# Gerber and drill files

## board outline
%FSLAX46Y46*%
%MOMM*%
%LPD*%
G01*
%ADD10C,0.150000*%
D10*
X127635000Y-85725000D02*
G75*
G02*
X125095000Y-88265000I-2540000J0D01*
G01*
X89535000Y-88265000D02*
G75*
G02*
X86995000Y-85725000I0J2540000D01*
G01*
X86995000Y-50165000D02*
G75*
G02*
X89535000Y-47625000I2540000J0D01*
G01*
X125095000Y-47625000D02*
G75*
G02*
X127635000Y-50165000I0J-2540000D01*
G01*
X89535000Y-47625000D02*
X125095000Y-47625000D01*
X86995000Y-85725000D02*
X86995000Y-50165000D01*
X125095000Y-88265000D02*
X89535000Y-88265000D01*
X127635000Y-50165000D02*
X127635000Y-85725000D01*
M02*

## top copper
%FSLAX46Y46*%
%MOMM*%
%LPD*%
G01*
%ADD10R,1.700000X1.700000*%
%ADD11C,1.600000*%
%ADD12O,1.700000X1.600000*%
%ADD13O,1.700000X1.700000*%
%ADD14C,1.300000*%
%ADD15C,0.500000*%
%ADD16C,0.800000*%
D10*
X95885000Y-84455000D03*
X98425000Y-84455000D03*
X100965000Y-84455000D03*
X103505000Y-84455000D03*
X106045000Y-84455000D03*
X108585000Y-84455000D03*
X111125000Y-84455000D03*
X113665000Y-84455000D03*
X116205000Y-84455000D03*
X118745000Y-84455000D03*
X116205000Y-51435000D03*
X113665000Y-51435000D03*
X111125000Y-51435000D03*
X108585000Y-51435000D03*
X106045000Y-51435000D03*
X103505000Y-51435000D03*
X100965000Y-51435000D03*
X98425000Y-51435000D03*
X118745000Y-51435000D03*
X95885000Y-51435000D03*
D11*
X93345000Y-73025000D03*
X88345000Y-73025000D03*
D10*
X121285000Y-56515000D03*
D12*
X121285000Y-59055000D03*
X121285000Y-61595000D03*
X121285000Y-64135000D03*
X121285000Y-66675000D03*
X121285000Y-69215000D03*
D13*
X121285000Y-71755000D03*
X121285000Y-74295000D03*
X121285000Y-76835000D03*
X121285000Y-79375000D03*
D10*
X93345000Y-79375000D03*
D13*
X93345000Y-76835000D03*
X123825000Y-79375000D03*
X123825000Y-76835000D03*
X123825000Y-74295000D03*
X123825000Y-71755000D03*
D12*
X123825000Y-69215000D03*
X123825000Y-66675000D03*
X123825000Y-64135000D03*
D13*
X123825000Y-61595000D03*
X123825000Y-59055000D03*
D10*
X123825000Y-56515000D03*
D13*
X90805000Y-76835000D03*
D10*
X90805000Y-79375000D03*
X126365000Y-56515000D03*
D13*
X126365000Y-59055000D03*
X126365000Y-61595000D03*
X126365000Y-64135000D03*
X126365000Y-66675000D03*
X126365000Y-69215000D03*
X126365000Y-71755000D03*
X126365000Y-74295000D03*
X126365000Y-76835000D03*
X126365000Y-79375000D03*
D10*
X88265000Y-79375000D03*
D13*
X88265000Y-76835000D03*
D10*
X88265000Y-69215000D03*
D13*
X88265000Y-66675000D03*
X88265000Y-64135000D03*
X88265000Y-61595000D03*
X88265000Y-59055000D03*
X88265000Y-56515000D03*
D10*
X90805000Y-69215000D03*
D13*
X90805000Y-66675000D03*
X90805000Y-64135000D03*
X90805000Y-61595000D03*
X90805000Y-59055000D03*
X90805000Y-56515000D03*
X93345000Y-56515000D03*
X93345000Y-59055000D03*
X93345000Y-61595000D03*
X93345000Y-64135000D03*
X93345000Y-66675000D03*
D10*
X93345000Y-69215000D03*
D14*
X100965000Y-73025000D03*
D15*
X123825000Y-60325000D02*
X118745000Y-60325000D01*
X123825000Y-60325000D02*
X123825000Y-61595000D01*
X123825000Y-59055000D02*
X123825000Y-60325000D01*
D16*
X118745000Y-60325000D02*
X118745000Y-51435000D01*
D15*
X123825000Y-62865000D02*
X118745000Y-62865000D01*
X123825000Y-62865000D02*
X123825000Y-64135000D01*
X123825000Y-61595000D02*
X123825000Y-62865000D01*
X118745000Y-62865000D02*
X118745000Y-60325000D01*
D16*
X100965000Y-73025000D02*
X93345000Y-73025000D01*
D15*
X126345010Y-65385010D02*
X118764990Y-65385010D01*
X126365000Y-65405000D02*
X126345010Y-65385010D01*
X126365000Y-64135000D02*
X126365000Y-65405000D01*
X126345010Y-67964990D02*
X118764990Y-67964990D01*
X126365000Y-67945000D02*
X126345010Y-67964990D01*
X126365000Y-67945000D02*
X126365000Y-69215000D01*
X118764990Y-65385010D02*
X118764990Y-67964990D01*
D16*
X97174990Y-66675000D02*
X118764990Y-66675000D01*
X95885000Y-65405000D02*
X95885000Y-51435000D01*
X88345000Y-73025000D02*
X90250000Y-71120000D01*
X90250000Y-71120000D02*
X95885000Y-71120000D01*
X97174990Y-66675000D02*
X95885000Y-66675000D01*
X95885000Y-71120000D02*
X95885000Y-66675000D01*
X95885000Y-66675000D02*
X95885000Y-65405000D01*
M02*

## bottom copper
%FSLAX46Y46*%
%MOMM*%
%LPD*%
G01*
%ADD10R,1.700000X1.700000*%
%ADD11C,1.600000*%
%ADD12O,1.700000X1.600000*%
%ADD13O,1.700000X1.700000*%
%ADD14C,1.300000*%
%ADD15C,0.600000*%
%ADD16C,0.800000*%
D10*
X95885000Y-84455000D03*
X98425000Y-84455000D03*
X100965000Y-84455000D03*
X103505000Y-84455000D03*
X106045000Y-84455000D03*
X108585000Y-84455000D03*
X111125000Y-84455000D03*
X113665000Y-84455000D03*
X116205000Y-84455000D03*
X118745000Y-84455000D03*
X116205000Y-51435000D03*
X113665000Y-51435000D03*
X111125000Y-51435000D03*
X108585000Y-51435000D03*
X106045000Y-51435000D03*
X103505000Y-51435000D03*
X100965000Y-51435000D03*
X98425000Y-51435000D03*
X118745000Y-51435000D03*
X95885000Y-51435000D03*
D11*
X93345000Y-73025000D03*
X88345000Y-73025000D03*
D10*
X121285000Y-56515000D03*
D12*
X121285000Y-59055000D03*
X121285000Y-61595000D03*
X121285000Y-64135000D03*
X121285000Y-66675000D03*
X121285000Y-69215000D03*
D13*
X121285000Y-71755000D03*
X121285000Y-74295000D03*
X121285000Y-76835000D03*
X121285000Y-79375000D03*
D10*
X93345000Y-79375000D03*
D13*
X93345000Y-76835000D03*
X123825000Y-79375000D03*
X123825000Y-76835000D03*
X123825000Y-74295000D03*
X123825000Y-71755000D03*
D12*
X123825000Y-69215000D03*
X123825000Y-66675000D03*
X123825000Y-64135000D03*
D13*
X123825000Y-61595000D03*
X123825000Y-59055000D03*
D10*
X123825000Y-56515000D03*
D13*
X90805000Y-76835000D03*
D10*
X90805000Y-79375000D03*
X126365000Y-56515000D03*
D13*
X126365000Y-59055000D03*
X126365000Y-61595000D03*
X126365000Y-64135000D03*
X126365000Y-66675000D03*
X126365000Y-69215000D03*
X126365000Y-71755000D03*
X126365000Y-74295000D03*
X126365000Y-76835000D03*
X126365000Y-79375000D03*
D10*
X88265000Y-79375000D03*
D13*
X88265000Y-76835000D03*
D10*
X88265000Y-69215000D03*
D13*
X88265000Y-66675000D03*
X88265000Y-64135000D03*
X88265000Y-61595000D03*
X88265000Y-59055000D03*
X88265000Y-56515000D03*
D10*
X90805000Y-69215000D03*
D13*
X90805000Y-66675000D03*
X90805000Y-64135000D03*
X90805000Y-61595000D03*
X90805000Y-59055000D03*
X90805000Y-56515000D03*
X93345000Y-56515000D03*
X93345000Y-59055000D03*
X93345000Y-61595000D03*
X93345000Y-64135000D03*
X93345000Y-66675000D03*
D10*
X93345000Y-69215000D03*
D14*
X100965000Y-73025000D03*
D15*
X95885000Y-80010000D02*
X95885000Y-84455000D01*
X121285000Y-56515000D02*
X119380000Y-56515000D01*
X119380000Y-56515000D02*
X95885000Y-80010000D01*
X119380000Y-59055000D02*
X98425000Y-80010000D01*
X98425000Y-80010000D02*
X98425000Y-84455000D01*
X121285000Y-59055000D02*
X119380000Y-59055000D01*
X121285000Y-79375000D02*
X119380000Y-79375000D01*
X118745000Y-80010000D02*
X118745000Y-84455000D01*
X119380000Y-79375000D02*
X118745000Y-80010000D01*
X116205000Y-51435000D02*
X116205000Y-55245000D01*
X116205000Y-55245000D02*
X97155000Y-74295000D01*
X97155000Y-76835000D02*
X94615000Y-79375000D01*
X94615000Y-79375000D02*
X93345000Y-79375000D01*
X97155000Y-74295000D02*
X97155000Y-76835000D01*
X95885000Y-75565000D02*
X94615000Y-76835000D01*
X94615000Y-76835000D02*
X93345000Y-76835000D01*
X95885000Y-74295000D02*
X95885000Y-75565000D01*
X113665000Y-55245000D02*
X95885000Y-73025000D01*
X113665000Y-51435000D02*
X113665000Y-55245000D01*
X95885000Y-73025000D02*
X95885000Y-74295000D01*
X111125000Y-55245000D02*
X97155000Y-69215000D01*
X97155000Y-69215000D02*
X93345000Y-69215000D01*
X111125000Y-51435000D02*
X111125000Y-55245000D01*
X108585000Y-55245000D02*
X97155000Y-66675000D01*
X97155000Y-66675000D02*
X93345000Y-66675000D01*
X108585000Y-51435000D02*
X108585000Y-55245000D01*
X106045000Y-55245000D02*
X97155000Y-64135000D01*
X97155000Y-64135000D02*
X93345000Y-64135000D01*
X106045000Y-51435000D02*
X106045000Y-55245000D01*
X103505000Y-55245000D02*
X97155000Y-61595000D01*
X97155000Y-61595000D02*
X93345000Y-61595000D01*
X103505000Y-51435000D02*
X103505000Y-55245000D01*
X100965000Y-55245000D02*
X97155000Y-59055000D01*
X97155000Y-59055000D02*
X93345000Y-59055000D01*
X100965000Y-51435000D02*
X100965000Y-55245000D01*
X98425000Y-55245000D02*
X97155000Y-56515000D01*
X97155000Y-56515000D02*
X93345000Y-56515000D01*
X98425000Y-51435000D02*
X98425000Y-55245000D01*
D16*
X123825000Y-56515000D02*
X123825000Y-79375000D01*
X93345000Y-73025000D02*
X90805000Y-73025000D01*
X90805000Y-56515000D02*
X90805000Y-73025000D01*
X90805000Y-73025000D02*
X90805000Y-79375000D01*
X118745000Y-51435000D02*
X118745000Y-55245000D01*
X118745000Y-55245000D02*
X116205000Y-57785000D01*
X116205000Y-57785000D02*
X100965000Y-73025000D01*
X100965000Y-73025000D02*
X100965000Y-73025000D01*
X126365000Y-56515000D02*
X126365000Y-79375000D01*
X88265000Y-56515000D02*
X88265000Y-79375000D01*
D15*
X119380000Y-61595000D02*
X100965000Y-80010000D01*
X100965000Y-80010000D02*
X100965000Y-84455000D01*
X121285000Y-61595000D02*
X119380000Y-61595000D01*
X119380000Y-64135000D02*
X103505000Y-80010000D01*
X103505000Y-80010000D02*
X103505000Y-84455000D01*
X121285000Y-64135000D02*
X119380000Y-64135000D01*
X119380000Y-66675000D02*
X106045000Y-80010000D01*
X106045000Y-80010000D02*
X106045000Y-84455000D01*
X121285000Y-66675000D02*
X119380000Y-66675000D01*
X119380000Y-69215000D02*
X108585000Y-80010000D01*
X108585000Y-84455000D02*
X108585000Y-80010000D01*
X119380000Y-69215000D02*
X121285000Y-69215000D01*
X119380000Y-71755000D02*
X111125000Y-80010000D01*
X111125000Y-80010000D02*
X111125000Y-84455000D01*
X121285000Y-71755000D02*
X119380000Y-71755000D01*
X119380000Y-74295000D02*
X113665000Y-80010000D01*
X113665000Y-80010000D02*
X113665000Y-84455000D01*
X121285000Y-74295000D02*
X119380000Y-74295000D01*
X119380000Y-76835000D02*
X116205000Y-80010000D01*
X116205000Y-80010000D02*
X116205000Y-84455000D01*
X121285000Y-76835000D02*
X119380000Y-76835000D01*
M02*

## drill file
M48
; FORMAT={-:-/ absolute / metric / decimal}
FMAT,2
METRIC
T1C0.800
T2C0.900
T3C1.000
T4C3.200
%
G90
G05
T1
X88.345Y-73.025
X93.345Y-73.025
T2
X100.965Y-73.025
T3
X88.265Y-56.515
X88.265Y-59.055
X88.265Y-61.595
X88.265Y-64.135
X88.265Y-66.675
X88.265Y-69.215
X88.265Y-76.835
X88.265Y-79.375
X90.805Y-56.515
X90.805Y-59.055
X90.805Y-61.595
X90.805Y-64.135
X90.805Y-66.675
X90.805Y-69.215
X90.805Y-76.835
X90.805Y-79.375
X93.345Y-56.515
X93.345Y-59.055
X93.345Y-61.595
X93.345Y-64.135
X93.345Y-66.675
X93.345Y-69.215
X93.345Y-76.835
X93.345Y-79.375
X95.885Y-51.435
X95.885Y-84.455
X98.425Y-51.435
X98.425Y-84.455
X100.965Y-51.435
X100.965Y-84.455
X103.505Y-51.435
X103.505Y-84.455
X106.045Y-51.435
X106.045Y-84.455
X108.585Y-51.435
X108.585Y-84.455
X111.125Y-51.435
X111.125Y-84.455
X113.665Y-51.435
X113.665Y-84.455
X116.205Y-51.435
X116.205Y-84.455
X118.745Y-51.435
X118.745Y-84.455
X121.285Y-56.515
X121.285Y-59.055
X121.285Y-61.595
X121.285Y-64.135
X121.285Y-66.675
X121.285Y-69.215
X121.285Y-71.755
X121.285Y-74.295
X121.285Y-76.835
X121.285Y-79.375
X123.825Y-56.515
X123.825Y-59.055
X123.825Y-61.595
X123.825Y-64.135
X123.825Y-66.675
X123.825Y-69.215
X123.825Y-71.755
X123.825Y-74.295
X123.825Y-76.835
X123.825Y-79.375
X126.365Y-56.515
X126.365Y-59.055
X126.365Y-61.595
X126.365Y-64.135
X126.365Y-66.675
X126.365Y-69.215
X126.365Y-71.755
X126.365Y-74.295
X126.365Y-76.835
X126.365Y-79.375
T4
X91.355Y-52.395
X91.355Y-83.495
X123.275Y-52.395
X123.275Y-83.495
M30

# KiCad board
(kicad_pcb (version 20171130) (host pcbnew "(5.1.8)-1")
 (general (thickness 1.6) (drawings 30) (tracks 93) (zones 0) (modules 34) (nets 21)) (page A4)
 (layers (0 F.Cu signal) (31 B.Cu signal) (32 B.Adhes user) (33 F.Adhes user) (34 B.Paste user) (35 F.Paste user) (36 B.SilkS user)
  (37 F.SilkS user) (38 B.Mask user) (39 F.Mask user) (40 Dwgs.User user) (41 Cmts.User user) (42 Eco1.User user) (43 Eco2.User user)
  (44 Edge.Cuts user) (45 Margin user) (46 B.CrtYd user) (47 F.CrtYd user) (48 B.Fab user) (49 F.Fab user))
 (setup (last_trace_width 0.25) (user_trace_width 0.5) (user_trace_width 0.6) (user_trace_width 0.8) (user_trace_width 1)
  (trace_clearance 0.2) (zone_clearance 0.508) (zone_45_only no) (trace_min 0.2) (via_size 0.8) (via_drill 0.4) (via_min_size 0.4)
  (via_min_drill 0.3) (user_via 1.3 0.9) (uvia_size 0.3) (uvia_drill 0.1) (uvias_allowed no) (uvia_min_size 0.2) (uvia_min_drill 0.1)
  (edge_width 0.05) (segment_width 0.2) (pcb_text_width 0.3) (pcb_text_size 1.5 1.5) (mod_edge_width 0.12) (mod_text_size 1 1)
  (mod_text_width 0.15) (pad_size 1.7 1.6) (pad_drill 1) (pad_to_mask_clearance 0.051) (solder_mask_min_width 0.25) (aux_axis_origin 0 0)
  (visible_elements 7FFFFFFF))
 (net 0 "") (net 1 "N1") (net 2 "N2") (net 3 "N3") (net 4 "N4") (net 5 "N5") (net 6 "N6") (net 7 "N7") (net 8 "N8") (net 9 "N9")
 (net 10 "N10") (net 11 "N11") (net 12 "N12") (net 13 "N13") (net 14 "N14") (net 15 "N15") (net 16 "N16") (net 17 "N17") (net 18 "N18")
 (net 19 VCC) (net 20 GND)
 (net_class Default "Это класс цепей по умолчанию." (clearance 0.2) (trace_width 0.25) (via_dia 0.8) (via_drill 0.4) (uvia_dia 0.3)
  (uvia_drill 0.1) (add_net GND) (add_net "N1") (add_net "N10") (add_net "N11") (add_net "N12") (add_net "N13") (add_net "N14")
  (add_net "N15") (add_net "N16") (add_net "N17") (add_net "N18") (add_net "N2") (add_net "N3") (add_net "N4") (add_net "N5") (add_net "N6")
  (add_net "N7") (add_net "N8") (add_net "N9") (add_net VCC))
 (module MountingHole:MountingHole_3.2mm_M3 (layer F.Cu) (at 123.2750 52.3950)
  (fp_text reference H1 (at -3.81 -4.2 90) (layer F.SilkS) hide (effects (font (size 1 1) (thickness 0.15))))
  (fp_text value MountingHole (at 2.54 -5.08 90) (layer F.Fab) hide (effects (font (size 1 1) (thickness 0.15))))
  (pad 1 np_thru_hole circle (at 0 0 270) (size 3.2 3.2) (drill 3.2) (layers *.Cu *.Mask)))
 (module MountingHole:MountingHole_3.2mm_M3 (layer F.Cu) (at 91.3550 52.3950)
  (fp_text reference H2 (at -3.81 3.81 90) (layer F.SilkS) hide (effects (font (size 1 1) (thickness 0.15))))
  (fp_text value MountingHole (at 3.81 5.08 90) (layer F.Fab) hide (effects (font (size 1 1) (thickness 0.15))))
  (pad 1 np_thru_hole circle (at 0 0 270) (size 3.2 3.2) (drill 3.2) (layers *.Cu *.Mask)))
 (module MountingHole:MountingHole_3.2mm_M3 (layer F.Cu) (at 123.2750 83.4950)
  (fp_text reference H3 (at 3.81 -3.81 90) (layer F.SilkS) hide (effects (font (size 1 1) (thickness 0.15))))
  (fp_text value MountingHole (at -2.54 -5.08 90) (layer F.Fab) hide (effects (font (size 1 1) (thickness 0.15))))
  (pad 1 np_thru_hole circle (at 0 0 270) (size 3.2 3.2) (drill 3.2) (layers *.Cu *.Mask)))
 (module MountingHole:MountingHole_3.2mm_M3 (layer F.Cu) (at 91.3550 83.4950)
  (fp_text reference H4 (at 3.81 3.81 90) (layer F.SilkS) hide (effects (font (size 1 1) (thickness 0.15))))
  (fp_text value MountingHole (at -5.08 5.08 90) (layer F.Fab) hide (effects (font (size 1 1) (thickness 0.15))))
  (pad 1 np_thru_hole circle (at 0 0 270) (size 3.2 3.2) (drill 3.2) (layers *.Cu *.Mask)))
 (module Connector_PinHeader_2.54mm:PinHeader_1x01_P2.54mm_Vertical (layer F.Cu) (at 95.885 84.455 270)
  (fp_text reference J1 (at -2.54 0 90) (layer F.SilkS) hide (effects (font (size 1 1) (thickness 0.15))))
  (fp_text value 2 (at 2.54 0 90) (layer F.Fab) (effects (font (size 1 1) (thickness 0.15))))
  (pad 1 thru_hole rect (at 0 0 270) (size 1.7 1.7) (drill 1) (layers *.Cu *.Mask) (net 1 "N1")))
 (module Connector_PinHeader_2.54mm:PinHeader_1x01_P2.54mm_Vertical (layer F.Cu) (at 98.425 84.455 270)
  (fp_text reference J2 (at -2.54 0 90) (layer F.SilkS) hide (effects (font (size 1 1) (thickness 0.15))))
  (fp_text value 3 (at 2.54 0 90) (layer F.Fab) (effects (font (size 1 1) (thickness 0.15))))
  (pad 1 thru_hole rect (at 0 0 270) (size 1.7 1.7) (drill 1) (layers *.Cu *.Mask) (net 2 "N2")))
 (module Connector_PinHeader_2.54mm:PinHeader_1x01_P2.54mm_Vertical (layer F.Cu) (at 100.965 84.455 270)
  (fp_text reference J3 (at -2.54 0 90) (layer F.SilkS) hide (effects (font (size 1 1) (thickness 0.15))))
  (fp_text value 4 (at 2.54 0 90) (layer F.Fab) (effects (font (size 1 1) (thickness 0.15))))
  (pad 1 thru_hole rect (at 0 0 270) (size 1.7 1.7) (drill 1) (layers *.Cu *.Mask) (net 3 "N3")))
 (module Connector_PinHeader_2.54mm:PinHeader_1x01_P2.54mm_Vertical (layer F.Cu) (at 103.505 84.455 270)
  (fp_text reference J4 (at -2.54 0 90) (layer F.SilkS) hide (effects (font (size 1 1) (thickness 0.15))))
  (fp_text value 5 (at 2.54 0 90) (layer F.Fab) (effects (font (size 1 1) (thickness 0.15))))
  (pad 1 thru_hole rect (at 0 0 270) (size 1.7 1.7) (drill 1) (layers *.Cu *.Mask) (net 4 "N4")))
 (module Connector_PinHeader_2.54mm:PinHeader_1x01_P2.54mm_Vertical (layer F.Cu) (at 106.045 84.455 270)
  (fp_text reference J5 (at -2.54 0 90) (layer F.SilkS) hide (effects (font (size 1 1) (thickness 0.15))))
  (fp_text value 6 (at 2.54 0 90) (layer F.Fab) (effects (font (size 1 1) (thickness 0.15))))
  (pad 1 thru_hole rect (at 0 0 270) (size 1.7 1.7) (drill 1) (layers *.Cu *.Mask) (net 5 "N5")))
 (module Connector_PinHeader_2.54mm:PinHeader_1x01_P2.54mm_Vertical (layer F.Cu) (at 108.585 84.455 270)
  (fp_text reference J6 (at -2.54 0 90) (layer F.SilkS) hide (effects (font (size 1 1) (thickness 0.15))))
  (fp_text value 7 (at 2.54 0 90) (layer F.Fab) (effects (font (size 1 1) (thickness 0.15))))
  (pad 1 thru_hole rect (at 0 0 270) (size 1.7 1.7) (drill 1) (layers *.Cu *.Mask) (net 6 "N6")))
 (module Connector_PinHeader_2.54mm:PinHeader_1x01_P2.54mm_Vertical (layer F.Cu) (at 111.125 84.455 270)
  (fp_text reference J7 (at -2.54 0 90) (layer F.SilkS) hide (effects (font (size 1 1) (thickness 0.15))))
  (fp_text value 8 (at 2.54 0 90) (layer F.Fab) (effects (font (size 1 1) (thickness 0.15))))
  (pad 1 thru_hole rect (at 0 0 270) (size 1.7 1.7) (drill 1) (layers *.Cu *.Mask) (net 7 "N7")))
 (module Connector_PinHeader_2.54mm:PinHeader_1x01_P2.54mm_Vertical (layer F.Cu) (at 113.665 84.455 270)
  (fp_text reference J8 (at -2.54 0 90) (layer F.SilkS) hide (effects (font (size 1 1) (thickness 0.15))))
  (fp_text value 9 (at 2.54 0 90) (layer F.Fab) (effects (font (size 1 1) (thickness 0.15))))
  (pad 1 thru_hole rect (at 0 0 270) (size 1.7 1.7) (drill 1) (layers *.Cu *.Mask) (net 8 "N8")))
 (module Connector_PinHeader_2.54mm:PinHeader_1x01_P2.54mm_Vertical (layer F.Cu) (at 116.205 84.455 270)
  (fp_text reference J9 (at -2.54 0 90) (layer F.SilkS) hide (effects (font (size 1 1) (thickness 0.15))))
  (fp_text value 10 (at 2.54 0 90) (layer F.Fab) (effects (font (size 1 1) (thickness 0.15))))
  (pad 1 thru_hole rect (at 0 0 270) (size 1.7 1.7) (drill 1) (layers *.Cu *.Mask) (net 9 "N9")))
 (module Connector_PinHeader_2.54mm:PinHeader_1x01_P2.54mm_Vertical (layer F.Cu) (at 118.745 84.455 270)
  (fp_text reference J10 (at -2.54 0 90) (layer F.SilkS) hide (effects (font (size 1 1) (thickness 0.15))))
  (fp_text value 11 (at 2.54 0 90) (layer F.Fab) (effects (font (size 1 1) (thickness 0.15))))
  (pad 1 thru_hole rect (at 0 0 270) (size 1.7 1.7) (drill 1) (layers *.Cu *.Mask) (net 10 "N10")))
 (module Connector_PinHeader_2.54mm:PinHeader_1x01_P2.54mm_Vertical (layer F.Cu) (at 116.205 51.435 270)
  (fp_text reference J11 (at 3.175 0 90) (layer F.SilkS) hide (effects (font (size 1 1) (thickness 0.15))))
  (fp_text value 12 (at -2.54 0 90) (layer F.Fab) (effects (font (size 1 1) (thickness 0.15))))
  (pad 1 thru_hole rect (at 0 0 270) (size 1.7 1.7) (drill 1) (layers *.Cu *.Mask) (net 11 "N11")))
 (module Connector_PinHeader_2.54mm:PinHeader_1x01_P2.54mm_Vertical (layer F.Cu) (at 113.665 51.435 270)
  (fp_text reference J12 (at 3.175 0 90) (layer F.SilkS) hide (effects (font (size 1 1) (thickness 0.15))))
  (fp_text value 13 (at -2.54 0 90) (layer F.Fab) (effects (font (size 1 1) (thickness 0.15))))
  (pad 1 thru_hole rect (at 0 0 270) (size 1.7 1.7) (drill 1) (layers *.Cu *.Mask) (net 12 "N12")))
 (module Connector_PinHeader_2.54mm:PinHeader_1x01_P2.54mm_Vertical (layer F.Cu) (at 111.125 51.435 270)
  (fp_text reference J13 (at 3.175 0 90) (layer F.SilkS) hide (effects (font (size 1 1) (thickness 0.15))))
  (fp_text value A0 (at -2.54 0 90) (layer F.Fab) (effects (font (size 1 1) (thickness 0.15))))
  (pad 1 thru_hole rect (at 0 0 270) (size 1.7 1.7) (drill 1) (layers *.Cu *.Mask) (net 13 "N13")))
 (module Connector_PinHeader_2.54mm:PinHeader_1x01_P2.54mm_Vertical (layer F.Cu) (at 108.585 51.435 270)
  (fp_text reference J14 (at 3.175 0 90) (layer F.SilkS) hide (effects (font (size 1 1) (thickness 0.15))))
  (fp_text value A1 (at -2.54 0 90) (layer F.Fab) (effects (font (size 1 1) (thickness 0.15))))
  (pad 1 thru_hole rect (at 0 0 270) (size 1.7 1.7) (drill 1) (layers *.Cu *.Mask) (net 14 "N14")))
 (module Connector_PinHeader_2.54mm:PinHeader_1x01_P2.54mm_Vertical (layer F.Cu) (at 106.045 51.435 270)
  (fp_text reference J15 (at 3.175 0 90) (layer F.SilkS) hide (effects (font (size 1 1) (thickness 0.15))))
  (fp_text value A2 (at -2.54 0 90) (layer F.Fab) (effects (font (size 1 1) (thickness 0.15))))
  (pad 1 thru_hole rect (at 0 0 270) (size 1.7 1.7) (drill 1) (layers *.Cu *.Mask) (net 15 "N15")))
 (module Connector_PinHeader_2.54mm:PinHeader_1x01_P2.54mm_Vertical (layer F.Cu) (at 103.505 51.435 270)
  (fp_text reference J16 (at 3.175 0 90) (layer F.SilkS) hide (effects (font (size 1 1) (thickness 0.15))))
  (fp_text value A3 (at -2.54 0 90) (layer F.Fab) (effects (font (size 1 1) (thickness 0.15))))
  (pad 1 thru_hole rect (at 0 0 270) (size 1.7 1.7) (drill 1) (layers *.Cu *.Mask) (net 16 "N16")))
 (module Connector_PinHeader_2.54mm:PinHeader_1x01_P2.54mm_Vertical (layer F.Cu) (at 100.965 51.435 270)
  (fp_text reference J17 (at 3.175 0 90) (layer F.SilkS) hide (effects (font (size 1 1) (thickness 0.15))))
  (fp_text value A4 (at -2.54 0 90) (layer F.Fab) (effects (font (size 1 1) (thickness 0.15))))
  (pad 1 thru_hole rect (at 0 0 270) (size 1.7 1.7) (drill 1) (layers *.Cu *.Mask) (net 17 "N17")))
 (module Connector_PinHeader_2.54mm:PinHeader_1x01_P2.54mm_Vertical (layer F.Cu) (at 98.425 51.435 270)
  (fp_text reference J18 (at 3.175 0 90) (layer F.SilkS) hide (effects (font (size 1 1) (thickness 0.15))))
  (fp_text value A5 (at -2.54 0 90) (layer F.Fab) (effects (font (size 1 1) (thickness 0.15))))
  (pad 1 thru_hole rect (at 0 0 270) (size 1.7 1.7) (drill 1) (layers *.Cu *.Mask) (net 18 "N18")))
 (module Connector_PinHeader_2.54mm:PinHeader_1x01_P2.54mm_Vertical (layer F.Cu) (at 118.745 51.435 270)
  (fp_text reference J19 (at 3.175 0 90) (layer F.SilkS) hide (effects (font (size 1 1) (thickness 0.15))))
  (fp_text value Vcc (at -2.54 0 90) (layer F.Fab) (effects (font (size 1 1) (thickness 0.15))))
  (pad 1 thru_hole rect (at 0 0 270) (size 1.7 1.7) (drill 1) (layers *.Cu *.Mask) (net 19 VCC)))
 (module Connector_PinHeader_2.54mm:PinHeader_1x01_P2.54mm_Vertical (layer F.Cu) (at 95.885 51.435 270)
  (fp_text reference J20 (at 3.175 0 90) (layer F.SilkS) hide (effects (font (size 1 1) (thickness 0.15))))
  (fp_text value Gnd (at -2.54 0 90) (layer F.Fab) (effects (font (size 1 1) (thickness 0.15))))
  (pad 1 thru_hole rect (at 0 0 270) (size 1.7 1.7) (drill 1) (layers *.Cu *.Mask) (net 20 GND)))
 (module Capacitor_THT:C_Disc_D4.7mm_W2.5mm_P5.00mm (layer F.Cu) (at 93.345 73.025 180)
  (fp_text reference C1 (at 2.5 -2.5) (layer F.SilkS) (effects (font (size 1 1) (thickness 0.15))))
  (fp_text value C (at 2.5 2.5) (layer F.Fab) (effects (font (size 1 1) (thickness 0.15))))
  (pad 1 thru_hole circle (at 0 0 180) (size 1.6 1.6) (drill 0.8) (layers *.Cu *.Mask) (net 19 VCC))
  (pad 2 thru_hole circle (at 5 0 180) (size 1.6 1.6) (drill 0.8) (layers *.Cu *.Mask) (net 20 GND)))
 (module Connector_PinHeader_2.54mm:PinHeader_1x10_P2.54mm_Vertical (layer F.Cu) (at 121.285 56.515)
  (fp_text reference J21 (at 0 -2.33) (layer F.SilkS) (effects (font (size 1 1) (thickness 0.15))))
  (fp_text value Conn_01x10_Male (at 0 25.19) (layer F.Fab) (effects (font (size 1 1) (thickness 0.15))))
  (pad 1 thru_hole rect (at 0 0) (size 1.7 1.7) (drill 1) (layers *.Cu *.Mask) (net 1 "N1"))
  (pad 2 thru_hole oval (at 0 2.54) (size 1.7 1.6) (drill 1) (layers *.Cu *.Mask) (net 2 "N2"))
  (pad 3 thru_hole oval (at 0 5.08) (size 1.7 1.6) (drill 1) (layers *.Cu *.Mask) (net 3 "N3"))
  (pad 4 thru_hole oval (at 0 7.62) (size 1.7 1.6) (drill 1) (layers *.Cu *.Mask) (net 4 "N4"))
  (pad 5 thru_hole oval (at 0 10.16) (size 1.7 1.6) (drill 1) (layers *.Cu *.Mask) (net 5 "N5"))
  (pad 6 thru_hole oval (at 0 12.7) (size 1.7 1.6) (drill 1) (layers *.Cu *.Mask) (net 6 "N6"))
  (pad 7 thru_hole oval (at 0 15.24) (size 1.7 1.7) (drill 1) (layers *.Cu *.Mask) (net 7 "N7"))
  (pad 8 thru_hole oval (at 0 17.78) (size 1.7 1.7) (drill 1) (layers *.Cu *.Mask) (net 8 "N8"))
  (pad 9 thru_hole oval (at 0 20.32) (size 1.7 1.7) (drill 1) (layers *.Cu *.Mask) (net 9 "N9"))
  (pad 10 thru_hole oval (at 0 22.86) (size 1.7 1.7) (drill 1) (layers *.Cu *.Mask) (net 10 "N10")))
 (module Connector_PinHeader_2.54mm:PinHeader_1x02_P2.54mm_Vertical (layer F.Cu) (at 93.345 79.375 180)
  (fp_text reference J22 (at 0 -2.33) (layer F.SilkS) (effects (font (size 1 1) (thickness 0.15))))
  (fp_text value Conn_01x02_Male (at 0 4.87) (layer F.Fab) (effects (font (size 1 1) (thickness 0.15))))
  (pad 1 thru_hole rect (at 0 0 180) (size 1.7 1.7) (drill 1) (layers *.Cu *.Mask) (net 11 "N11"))
  (pad 2 thru_hole oval (at 0 2.54 180) (size 1.7 1.7) (drill 1) (layers *.Cu *.Mask) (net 12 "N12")))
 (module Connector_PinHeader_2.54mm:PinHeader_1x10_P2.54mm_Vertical (layer F.Cu) (at 123.825 56.515)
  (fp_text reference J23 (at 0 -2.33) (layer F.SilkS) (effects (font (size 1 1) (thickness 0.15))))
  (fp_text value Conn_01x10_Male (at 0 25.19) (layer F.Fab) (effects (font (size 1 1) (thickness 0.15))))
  (pad 10 thru_hole oval (at 0 22.86) (size 1.7 1.7) (drill 1) (layers *.Cu *.Mask) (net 19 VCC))
  (pad 9 thru_hole oval (at 0 20.32) (size 1.7 1.7) (drill 1) (layers *.Cu *.Mask) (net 19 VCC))
  (pad 8 thru_hole oval (at 0 17.78) (size 1.7 1.7) (drill 1) (layers *.Cu *.Mask) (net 19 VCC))
  (pad 7 thru_hole oval (at 0 15.24) (size 1.7 1.7) (drill 1) (layers *.Cu *.Mask) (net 19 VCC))
  (pad 6 thru_hole oval (at 0 12.7) (size 1.7 1.6) (drill 1) (layers *.Cu *.Mask) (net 19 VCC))
  (pad 5 thru_hole oval (at 0 10.16) (size 1.7 1.6) (drill 1) (layers *.Cu *.Mask) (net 19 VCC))
  (pad 4 thru_hole oval (at 0 7.62) (size 1.7 1.6) (drill 1) (layers *.Cu *.Mask) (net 19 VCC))
  (pad 3 thru_hole oval (at 0 5.08) (size 1.7 1.7) (drill 1) (layers *.Cu *.Mask) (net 19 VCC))
  (pad 2 thru_hole oval (at 0 2.54) (size 1.7 1.7) (drill 1) (layers *.Cu *.Mask) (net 19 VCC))
  (pad 1 thru_hole rect (at 0 0) (size 1.7 1.7) (drill 1) (layers *.Cu *.Mask) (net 19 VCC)))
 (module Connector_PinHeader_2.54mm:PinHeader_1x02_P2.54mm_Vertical (layer F.Cu) (at 90.805 79.375 180)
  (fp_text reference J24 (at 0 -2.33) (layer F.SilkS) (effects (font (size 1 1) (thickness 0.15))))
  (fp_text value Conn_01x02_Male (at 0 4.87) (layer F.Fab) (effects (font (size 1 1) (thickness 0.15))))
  (pad 2 thru_hole oval (at 0 2.54 180) (size 1.7 1.7) (drill 1) (layers *.Cu *.Mask) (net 19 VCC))
  (pad 1 thru_hole rect (at 0 0 180) (size 1.7 1.7) (drill 1) (layers *.Cu *.Mask) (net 19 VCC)))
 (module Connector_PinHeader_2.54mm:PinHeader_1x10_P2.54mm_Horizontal (layer F.Cu) (at 126.365 56.515)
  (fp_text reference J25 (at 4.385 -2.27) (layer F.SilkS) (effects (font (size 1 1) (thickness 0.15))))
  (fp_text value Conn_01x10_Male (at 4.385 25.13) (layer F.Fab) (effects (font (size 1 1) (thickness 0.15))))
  (pad 1 thru_hole rect (at 0 0) (size 1.7 1.7) (drill 1) (layers *.Cu *.Mask) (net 20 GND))
  (pad 2 thru_hole oval (at 0 2.54) (size 1.7 1.7) (drill 1) (layers *.Cu *.Mask) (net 20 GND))
  (pad 3 thru_hole oval (at 0 5.08) (size 1.7 1.7) (drill 1) (layers *.Cu *.Mask) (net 20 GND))
  (pad 4 thru_hole oval (at 0 7.62) (size 1.7 1.7) (drill 1) (layers *.Cu *.Mask) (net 20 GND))
  (pad 5 thru_hole oval (at 0 10.16) (size 1.7 1.7) (drill 1) (layers *.Cu *.Mask) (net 20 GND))
  (pad 6 thru_hole oval (at 0 12.7) (size 1.7 1.7) (drill 1) (layers *.Cu *.Mask) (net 20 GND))
  (pad 7 thru_hole oval (at 0 15.24) (size 1.7 1.7) (drill 1) (layers *.Cu *.Mask) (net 20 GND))
  (pad 8 thru_hole oval (at 0 17.78) (size 1.7 1.7) (drill 1) (layers *.Cu *.Mask) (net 20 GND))
  (pad 9 thru_hole oval (at 0 20.32) (size 1.7 1.7) (drill 1) (layers *.Cu *.Mask) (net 20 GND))
  (pad 10 thru_hole oval (at 0 22.86) (size 1.7 1.7) (drill 1) (layers *.Cu *.Mask) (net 20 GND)))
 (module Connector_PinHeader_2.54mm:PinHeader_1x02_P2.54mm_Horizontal (layer F.Cu) (at 88.265 79.375 180)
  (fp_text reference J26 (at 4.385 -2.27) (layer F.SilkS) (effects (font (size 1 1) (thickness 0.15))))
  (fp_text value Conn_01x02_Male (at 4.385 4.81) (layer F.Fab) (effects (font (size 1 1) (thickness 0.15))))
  (pad 1 thru_hole rect (at 0 0 180) (size 1.7 1.7) (drill 1) (layers *.Cu *.Mask) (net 20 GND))
  (pad 2 thru_hole oval (at 0 2.54 180) (size 1.7 1.7) (drill 1) (layers *.Cu *.Mask) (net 20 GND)))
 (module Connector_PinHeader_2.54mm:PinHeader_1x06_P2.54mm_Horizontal (layer F.Cu) (at 88.265 69.215 180)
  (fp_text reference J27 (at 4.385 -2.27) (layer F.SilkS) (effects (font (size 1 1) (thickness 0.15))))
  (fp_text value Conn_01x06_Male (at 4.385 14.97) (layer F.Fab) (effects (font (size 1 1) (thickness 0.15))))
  (pad 1 thru_hole rect (at 0 0 180) (size 1.7 1.7) (drill 1) (layers *.Cu *.Mask) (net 20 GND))
  (pad 2 thru_hole oval (at 0 2.54 180) (size 1.7 1.7) (drill 1) (layers *.Cu *.Mask) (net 20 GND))
  (pad 3 thru_hole oval (at 0 5.08 180) (size 1.7 1.7) (drill 1) (layers *.Cu *.Mask) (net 20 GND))
  (pad 4 thru_hole oval (at 0 7.62 180) (size 1.7 1.7) (drill 1) (layers *.Cu *.Mask) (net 20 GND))
  (pad 5 thru_hole oval (at 0 10.16 180) (size 1.7 1.7) (drill 1) (layers *.Cu *.Mask) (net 20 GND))
  (pad 6 thru_hole oval (at 0 12.7 180) (size 1.7 1.7) (drill 1) (layers *.Cu *.Mask) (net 20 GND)))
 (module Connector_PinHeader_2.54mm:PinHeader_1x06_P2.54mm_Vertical (layer F.Cu) (at 90.805 69.215 180)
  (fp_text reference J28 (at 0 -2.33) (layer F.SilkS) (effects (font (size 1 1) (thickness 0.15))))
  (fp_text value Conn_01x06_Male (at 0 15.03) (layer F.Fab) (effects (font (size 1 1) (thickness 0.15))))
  (pad 1 thru_hole rect (at 0 0 180) (size 1.7 1.7) (drill 1) (layers *.Cu *.Mask) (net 19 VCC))
  (pad 2 thru_hole oval (at 0 2.54 180) (size 1.7 1.7) (drill 1) (layers *.Cu *.Mask) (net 19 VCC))
  (pad 3 thru_hole oval (at 0 5.08 180) (size 1.7 1.7) (drill 1) (layers *.Cu *.Mask) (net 19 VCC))
  (pad 4 thru_hole oval (at 0 7.62 180) (size 1.7 1.7) (drill 1) (layers *.Cu *.Mask) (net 19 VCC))
  (pad 5 thru_hole oval (at 0 10.16 180) (size 1.7 1.7) (drill 1) (layers *.Cu *.Mask) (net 19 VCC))
  (pad 6 thru_hole oval (at 0 12.7 180) (size 1.7 1.7) (drill 1) (layers *.Cu *.Mask) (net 19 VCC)))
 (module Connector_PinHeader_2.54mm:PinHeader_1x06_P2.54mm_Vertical (layer F.Cu) (at 93.345 69.215 180)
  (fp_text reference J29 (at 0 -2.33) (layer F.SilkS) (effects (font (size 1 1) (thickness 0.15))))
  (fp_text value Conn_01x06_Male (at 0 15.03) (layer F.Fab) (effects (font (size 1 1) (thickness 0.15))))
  (pad 6 thru_hole oval (at 0 12.7 180) (size 1.7 1.7) (drill 1) (layers *.Cu *.Mask) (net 18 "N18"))
  (pad 5 thru_hole oval (at 0 10.16 180) (size 1.7 1.7) (drill 1) (layers *.Cu *.Mask) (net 17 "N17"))
  (pad 4 thru_hole oval (at 0 7.62 180) (size 1.7 1.7) (drill 1) (layers *.Cu *.Mask) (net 16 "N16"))
  (pad 3 thru_hole oval (at 0 5.08 180) (size 1.7 1.7) (drill 1) (layers *.Cu *.Mask) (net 15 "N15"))
  (pad 2 thru_hole oval (at 0 2.54 180) (size 1.7 1.7) (drill 1) (layers *.Cu *.Mask) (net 14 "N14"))
  (pad 1 thru_hole rect (at 0 0 180) (size 1.7 1.7) (drill 1) (layers *.Cu *.Mask) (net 13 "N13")))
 (gr_arc (start 125.095 85.725) (end 125.095 88.265) (angle -90) (layer Edge.Cuts) (width 0.15))
 (gr_arc (start 89.535 85.725) (end 86.995 85.725) (angle -90) (layer Edge.Cuts) (width 0.15))
 (gr_arc (start 89.535 50.165) (end 89.535 47.625) (angle -90) (layer Edge.Cuts) (width 0.15))
 (gr_arc (start 125.095 50.165) (end 127.635 50.165) (angle -90) (layer Edge.Cuts) (width 0.15))
 (gr_line (start 89.535 47.625) (end 125.095 47.625) (layer Edge.Cuts) (width 0.15))
 (gr_line (start 86.995 85.725) (end 86.995 50.165) (layer Edge.Cuts) (width 0.15))
 (gr_line (start 125.095 88.265) (end 89.535 88.265) (layer Edge.Cuts) (width 0.15))
 (gr_line (start 127.635 50.165) (end 127.635 85.725) (layer Edge.Cuts) (width 0.15))
 (segment (start 95.885 80.01) (end 95.885 84.455) (width 0.6) (layer B.Cu) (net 1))
 (segment (start 121.285 56.515) (end 119.38 56.515) (width 0.6) (layer B.Cu) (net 1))
 (segment (start 119.38 56.515) (end 95.885 80.01) (width 0.6) (layer B.Cu) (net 1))
 (segment (start 119.38 59.055) (end 98.425 80.01) (width 0.6) (layer B.Cu) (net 2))
 (segment (start 98.425 80.01) (end 98.425 84.455) (width 0.6) (layer B.Cu) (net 2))
 (segment (start 121.285 59.055) (end 119.38 59.055) (width 0.6) (layer B.Cu) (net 2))
 (segment (start 121.285 79.375) (end 119.38 79.375) (width 0.6) (layer B.Cu) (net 10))
 (segment (start 118.745 80.01) (end 118.745 84.455) (width 0.6) (layer B.Cu) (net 10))
 (segment (start 119.38 79.375) (end 118.745 80.01) (width 0.6) (layer B.Cu) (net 10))
 (segment (start 116.205 51.435) (end 116.205 55.245) (width 0.6) (layer B.Cu) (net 11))
 (segment (start 116.205 55.245) (end 97.155 74.295) (width 0.6) (layer B.Cu) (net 11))
 (segment (start 97.155 76.835) (end 94.615 79.375) (width 0.6) (layer B.Cu) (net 11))
 (segment (start 94.615 79.375) (end 93.345 79.375) (width 0.6) (layer B.Cu) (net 11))
 (segment (start 97.155 74.295) (end 97.155 76.835) (width 0.6) (layer B.Cu) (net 11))
 (segment (start 95.885 75.565) (end 94.615 76.835) (width 0.6) (layer B.Cu) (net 12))
 (segment (start 94.615 76.835) (end 93.345 76.835) (width 0.6) (layer B.Cu) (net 12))
 (segment (start 95.885 74.295) (end 95.885 75.565) (width 0.6) (layer B.Cu) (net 12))
 (segment (start 113.665 55.245) (end 95.885 73.025) (width 0.6) (layer B.Cu) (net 12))
 (segment (start 113.665 51.435) (end 113.665 55.245) (width 0.6) (layer B.Cu) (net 12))
 (segment (start 95.885 73.025) (end 95.885 74.295) (width 0.6) (layer B.Cu) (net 12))
 (segment (start 111.125 55.245) (end 97.155 69.215) (width 0.6) (layer B.Cu) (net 13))
 (segment (start 97.155 69.215) (end 93.345 69.215) (width 0.6) (layer B.Cu) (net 13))
 (segment (start 111.125 51.435) (end 111.125 55.245) (width 0.6) (layer B.Cu) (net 13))
 (segment (start 108.585 55.245) (end 97.155 66.675) (width 0.6) (layer B.Cu) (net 14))
 (segment (start 97.155 66.675) (end 93.345 66.675) (width 0.6) (layer B.Cu) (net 14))
 (segment (start 108.585 51.435) (end 108.585 55.245) (width 0.6) (layer B.Cu) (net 14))
 (segment (start 106.045 55.245) (end 97.155 64.135) (width 0.6) (layer B.Cu) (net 15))
 (segment (start 97.155 64.135) (end 93.345 64.135) (width 0.6) (layer B.Cu) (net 15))
 (segment (start 106.045 51.435) (end 106.045 55.245) (width 0.6) (layer B.Cu) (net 15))
 (segment (start 103.505 55.245) (end 97.155 61.595) (width 0.6) (layer B.Cu) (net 16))
 (segment (start 97.155 61.595) (end 93.345 61.595) (width 0.6) (layer B.Cu) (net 16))
 (segment (start 103.505 51.435) (end 103.505 55.245) (width 0.6) (layer B.Cu) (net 16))
 (segment (start 100.965 55.245) (end 97.155 59.055) (width 0.6) (layer B.Cu) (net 17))
 (segment (start 97.155 59.055) (end 93.345 59.055) (width 0.6) (layer B.Cu) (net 17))
 (segment (start 100.965 51.435) (end 100.965 55.245) (width 0.6) (layer B.Cu) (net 17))
 (segment (start 98.425 55.245) (end 97.155 56.515) (width 0.6) (layer B.Cu) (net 18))
 (segment (start 97.155 56.515) (end 93.345 56.515) (width 0.6) (layer B.Cu) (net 18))
 (segment (start 98.425 51.435) (end 98.425 55.245) (width 0.6) (layer B.Cu) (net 18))
 (segment (start 123.825 56.515) (end 123.825 79.375) (width 0.8) (layer B.Cu) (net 19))
 (segment (start 93.345 73.025) (end 90.805 73.025) (width 0.8) (layer B.Cu) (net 19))
 (segment (start 90.805 56.515) (end 90.805 73.025) (width 0.8) (layer B.Cu) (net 19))
 (segment (start 90.805 73.025) (end 90.805 79.375) (width 0.8) (layer B.Cu) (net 19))
 (segment (start 123.825 60.325) (end 118.745 60.325) (width 0.5) (layer F.Cu) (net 19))
 (segment (start 123.825 60.325) (end 123.825 61.595) (width 0.5) (layer F.Cu) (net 19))
 (segment (start 123.825 59.055) (end 123.825 60.325) (width 0.5) (layer F.Cu) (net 19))
 (segment (start 118.745 60.325) (end 118.745 51.435) (width 0.8) (layer F.Cu) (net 19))
 (segment (start 123.825 62.865) (end 118.745 62.865) (width 0.5) (layer F.Cu) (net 19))
 (segment (start 123.825 62.865) (end 123.825 64.135) (width 0.5) (layer F.Cu) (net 19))
 (segment (start 123.825 61.595) (end 123.825 62.865) (width 0.5) (layer F.Cu) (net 19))
 (segment (start 118.745 62.865) (end 118.745 60.325) (width 0.5) (layer F.Cu) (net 19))
 (segment (start 118.745 51.435) (end 118.745 55.245) (width 0.8) (layer B.Cu) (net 19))
 (segment (start 118.745 55.245) (end 116.205 57.785) (width 0.8) (layer B.Cu) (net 19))
 (segment (start 116.205 57.785) (end 100.965 73.025) (width 0.8) (layer B.Cu) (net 19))
 (segment (start 100.965 73.025) (end 100.965 73.025) (width 0.8) (layer B.Cu) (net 19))
 (via (at 100.965 73.025) (size 1.3) (drill 0.9) (layers F.Cu B.Cu) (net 19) (status 1000000))
 (segment (start 100.965 73.025) (end 93.345 73.025) (width 0.8) (layer F.Cu) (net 19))
 (segment (start 126.365 56.515) (end 126.365 79.375) (width 0.8) (layer B.Cu) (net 20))
 (segment (start 88.265 56.515) (end 88.265 79.375) (width 0.8) (layer B.Cu) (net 20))
 (segment (start 126.34501 65.38501) (end 118.76499 65.38501) (width 0.5) (layer F.Cu) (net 20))
 (segment (start 126.365 65.405) (end 126.34501 65.38501) (width 0.5) (layer F.Cu) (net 20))
 (segment (start 126.365 64.135) (end 126.365 65.405) (width 0.5) (layer F.Cu) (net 20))
 (segment (start 126.34501 67.96499) (end 118.76499 67.96499) (width 0.5) (layer F.Cu) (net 20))
 (segment (start 126.365 67.945) (end 126.34501 67.96499) (width 0.5) (layer F.Cu) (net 20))
 (segment (start 126.365 67.945) (end 126.365 69.215) (width 0.5) (layer F.Cu) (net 20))
 (segment (start 118.76499 65.38501) (end 118.76499 67.96499) (width 0.5) (layer F.Cu) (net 20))
 (segment (start 97.17499 66.675) (end 118.76499 66.675) (width 0.8) (layer F.Cu) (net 20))
 (segment (start 95.885 65.405) (end 95.885 51.435) (width 0.8) (layer F.Cu) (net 20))
 (segment (start 88.345 73.025) (end 90.25 71.12) (width 0.8) (layer F.Cu) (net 20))
 (segment (start 90.25 71.12) (end 95.885 71.12) (width 0.8) (layer F.Cu) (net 20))
 (segment (start 97.17499 66.675) (end 95.885 66.675) (width 0.8) (layer F.Cu) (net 20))
 (segment (start 95.885 71.12) (end 95.885 66.675) (width 0.8) (layer F.Cu) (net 20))
 (segment (start 95.885 66.675) (end 95.885 65.405) (width 0.8) (layer F.Cu) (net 20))
 (segment (start 119.38 61.595) (end 100.965 80.01) (width 0.6) (layer B.Cu) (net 3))
 (segment (start 100.965 80.01) (end 100.965 84.455) (width 0.6) (layer B.Cu) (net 3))
 (segment (start 121.285 61.595) (end 119.38 61.595) (width 0.6) (layer B.Cu) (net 3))
 (segment (start 119.38 64.135) (end 103.505 80.01) (width 0.6) (layer B.Cu) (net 4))
 (segment (start 103.505 80.01) (end 103.505 84.455) (width 0.6) (layer B.Cu) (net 4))
 (segment (start 121.285 64.135) (end 119.38 64.135) (width 0.6) (layer B.Cu) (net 4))
 (segment (start 119.38 66.675) (end 106.045 80.01) (width 0.6) (layer B.Cu) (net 5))
 (segment (start 106.045 80.01) (end 106.045 84.455) (width 0.6) (layer B.Cu) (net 5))
 (segment (start 121.285 66.675) (end 119.38 66.675) (width 0.6) (layer B.Cu) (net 5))
 (segment (start 119.38 69.215) (end 108.585 80.01) (width 0.6) (layer B.Cu) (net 6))
 (segment (start 108.585 84.455) (end 108.585 80.01) (width 0.6) (layer B.Cu) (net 6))
 (segment (start 119.38 69.215) (end 121.285 69.215) (width 0.6) (layer B.Cu) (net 6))
 (segment (start 119.38 71.755) (end 111.125 80.01) (width 0.6) (layer B.Cu) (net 7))
 (segment (start 111.125 80.01) (end 111.125 84.455) (width 0.6) (layer B.Cu) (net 7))
 (segment (start 121.285 71.755) (end 119.38 71.755) (width 0.6) (layer B.Cu) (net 7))
 (segment (start 119.38 74.295) (end 113.665 80.01) (width 0.6) (layer B.Cu) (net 8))
 (segment (start 113.665 80.01) (end 113.665 84.455) (width 0.6) (layer B.Cu) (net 8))
 (segment (start 121.285 74.295) (end 119.38 74.295) (width 0.6) (layer B.Cu) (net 8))
 (segment (start 119.38 76.835) (end 116.205 80.01) (width 0.6) (layer B.Cu) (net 9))
 (segment (start 116.205 80.01) (end 116.205 84.455) (width 0.6) (layer B.Cu) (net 9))
 (segment (start 121.285 76.835) (end 119.38 76.835) (width 0.6) (layer B.Cu) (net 9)))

